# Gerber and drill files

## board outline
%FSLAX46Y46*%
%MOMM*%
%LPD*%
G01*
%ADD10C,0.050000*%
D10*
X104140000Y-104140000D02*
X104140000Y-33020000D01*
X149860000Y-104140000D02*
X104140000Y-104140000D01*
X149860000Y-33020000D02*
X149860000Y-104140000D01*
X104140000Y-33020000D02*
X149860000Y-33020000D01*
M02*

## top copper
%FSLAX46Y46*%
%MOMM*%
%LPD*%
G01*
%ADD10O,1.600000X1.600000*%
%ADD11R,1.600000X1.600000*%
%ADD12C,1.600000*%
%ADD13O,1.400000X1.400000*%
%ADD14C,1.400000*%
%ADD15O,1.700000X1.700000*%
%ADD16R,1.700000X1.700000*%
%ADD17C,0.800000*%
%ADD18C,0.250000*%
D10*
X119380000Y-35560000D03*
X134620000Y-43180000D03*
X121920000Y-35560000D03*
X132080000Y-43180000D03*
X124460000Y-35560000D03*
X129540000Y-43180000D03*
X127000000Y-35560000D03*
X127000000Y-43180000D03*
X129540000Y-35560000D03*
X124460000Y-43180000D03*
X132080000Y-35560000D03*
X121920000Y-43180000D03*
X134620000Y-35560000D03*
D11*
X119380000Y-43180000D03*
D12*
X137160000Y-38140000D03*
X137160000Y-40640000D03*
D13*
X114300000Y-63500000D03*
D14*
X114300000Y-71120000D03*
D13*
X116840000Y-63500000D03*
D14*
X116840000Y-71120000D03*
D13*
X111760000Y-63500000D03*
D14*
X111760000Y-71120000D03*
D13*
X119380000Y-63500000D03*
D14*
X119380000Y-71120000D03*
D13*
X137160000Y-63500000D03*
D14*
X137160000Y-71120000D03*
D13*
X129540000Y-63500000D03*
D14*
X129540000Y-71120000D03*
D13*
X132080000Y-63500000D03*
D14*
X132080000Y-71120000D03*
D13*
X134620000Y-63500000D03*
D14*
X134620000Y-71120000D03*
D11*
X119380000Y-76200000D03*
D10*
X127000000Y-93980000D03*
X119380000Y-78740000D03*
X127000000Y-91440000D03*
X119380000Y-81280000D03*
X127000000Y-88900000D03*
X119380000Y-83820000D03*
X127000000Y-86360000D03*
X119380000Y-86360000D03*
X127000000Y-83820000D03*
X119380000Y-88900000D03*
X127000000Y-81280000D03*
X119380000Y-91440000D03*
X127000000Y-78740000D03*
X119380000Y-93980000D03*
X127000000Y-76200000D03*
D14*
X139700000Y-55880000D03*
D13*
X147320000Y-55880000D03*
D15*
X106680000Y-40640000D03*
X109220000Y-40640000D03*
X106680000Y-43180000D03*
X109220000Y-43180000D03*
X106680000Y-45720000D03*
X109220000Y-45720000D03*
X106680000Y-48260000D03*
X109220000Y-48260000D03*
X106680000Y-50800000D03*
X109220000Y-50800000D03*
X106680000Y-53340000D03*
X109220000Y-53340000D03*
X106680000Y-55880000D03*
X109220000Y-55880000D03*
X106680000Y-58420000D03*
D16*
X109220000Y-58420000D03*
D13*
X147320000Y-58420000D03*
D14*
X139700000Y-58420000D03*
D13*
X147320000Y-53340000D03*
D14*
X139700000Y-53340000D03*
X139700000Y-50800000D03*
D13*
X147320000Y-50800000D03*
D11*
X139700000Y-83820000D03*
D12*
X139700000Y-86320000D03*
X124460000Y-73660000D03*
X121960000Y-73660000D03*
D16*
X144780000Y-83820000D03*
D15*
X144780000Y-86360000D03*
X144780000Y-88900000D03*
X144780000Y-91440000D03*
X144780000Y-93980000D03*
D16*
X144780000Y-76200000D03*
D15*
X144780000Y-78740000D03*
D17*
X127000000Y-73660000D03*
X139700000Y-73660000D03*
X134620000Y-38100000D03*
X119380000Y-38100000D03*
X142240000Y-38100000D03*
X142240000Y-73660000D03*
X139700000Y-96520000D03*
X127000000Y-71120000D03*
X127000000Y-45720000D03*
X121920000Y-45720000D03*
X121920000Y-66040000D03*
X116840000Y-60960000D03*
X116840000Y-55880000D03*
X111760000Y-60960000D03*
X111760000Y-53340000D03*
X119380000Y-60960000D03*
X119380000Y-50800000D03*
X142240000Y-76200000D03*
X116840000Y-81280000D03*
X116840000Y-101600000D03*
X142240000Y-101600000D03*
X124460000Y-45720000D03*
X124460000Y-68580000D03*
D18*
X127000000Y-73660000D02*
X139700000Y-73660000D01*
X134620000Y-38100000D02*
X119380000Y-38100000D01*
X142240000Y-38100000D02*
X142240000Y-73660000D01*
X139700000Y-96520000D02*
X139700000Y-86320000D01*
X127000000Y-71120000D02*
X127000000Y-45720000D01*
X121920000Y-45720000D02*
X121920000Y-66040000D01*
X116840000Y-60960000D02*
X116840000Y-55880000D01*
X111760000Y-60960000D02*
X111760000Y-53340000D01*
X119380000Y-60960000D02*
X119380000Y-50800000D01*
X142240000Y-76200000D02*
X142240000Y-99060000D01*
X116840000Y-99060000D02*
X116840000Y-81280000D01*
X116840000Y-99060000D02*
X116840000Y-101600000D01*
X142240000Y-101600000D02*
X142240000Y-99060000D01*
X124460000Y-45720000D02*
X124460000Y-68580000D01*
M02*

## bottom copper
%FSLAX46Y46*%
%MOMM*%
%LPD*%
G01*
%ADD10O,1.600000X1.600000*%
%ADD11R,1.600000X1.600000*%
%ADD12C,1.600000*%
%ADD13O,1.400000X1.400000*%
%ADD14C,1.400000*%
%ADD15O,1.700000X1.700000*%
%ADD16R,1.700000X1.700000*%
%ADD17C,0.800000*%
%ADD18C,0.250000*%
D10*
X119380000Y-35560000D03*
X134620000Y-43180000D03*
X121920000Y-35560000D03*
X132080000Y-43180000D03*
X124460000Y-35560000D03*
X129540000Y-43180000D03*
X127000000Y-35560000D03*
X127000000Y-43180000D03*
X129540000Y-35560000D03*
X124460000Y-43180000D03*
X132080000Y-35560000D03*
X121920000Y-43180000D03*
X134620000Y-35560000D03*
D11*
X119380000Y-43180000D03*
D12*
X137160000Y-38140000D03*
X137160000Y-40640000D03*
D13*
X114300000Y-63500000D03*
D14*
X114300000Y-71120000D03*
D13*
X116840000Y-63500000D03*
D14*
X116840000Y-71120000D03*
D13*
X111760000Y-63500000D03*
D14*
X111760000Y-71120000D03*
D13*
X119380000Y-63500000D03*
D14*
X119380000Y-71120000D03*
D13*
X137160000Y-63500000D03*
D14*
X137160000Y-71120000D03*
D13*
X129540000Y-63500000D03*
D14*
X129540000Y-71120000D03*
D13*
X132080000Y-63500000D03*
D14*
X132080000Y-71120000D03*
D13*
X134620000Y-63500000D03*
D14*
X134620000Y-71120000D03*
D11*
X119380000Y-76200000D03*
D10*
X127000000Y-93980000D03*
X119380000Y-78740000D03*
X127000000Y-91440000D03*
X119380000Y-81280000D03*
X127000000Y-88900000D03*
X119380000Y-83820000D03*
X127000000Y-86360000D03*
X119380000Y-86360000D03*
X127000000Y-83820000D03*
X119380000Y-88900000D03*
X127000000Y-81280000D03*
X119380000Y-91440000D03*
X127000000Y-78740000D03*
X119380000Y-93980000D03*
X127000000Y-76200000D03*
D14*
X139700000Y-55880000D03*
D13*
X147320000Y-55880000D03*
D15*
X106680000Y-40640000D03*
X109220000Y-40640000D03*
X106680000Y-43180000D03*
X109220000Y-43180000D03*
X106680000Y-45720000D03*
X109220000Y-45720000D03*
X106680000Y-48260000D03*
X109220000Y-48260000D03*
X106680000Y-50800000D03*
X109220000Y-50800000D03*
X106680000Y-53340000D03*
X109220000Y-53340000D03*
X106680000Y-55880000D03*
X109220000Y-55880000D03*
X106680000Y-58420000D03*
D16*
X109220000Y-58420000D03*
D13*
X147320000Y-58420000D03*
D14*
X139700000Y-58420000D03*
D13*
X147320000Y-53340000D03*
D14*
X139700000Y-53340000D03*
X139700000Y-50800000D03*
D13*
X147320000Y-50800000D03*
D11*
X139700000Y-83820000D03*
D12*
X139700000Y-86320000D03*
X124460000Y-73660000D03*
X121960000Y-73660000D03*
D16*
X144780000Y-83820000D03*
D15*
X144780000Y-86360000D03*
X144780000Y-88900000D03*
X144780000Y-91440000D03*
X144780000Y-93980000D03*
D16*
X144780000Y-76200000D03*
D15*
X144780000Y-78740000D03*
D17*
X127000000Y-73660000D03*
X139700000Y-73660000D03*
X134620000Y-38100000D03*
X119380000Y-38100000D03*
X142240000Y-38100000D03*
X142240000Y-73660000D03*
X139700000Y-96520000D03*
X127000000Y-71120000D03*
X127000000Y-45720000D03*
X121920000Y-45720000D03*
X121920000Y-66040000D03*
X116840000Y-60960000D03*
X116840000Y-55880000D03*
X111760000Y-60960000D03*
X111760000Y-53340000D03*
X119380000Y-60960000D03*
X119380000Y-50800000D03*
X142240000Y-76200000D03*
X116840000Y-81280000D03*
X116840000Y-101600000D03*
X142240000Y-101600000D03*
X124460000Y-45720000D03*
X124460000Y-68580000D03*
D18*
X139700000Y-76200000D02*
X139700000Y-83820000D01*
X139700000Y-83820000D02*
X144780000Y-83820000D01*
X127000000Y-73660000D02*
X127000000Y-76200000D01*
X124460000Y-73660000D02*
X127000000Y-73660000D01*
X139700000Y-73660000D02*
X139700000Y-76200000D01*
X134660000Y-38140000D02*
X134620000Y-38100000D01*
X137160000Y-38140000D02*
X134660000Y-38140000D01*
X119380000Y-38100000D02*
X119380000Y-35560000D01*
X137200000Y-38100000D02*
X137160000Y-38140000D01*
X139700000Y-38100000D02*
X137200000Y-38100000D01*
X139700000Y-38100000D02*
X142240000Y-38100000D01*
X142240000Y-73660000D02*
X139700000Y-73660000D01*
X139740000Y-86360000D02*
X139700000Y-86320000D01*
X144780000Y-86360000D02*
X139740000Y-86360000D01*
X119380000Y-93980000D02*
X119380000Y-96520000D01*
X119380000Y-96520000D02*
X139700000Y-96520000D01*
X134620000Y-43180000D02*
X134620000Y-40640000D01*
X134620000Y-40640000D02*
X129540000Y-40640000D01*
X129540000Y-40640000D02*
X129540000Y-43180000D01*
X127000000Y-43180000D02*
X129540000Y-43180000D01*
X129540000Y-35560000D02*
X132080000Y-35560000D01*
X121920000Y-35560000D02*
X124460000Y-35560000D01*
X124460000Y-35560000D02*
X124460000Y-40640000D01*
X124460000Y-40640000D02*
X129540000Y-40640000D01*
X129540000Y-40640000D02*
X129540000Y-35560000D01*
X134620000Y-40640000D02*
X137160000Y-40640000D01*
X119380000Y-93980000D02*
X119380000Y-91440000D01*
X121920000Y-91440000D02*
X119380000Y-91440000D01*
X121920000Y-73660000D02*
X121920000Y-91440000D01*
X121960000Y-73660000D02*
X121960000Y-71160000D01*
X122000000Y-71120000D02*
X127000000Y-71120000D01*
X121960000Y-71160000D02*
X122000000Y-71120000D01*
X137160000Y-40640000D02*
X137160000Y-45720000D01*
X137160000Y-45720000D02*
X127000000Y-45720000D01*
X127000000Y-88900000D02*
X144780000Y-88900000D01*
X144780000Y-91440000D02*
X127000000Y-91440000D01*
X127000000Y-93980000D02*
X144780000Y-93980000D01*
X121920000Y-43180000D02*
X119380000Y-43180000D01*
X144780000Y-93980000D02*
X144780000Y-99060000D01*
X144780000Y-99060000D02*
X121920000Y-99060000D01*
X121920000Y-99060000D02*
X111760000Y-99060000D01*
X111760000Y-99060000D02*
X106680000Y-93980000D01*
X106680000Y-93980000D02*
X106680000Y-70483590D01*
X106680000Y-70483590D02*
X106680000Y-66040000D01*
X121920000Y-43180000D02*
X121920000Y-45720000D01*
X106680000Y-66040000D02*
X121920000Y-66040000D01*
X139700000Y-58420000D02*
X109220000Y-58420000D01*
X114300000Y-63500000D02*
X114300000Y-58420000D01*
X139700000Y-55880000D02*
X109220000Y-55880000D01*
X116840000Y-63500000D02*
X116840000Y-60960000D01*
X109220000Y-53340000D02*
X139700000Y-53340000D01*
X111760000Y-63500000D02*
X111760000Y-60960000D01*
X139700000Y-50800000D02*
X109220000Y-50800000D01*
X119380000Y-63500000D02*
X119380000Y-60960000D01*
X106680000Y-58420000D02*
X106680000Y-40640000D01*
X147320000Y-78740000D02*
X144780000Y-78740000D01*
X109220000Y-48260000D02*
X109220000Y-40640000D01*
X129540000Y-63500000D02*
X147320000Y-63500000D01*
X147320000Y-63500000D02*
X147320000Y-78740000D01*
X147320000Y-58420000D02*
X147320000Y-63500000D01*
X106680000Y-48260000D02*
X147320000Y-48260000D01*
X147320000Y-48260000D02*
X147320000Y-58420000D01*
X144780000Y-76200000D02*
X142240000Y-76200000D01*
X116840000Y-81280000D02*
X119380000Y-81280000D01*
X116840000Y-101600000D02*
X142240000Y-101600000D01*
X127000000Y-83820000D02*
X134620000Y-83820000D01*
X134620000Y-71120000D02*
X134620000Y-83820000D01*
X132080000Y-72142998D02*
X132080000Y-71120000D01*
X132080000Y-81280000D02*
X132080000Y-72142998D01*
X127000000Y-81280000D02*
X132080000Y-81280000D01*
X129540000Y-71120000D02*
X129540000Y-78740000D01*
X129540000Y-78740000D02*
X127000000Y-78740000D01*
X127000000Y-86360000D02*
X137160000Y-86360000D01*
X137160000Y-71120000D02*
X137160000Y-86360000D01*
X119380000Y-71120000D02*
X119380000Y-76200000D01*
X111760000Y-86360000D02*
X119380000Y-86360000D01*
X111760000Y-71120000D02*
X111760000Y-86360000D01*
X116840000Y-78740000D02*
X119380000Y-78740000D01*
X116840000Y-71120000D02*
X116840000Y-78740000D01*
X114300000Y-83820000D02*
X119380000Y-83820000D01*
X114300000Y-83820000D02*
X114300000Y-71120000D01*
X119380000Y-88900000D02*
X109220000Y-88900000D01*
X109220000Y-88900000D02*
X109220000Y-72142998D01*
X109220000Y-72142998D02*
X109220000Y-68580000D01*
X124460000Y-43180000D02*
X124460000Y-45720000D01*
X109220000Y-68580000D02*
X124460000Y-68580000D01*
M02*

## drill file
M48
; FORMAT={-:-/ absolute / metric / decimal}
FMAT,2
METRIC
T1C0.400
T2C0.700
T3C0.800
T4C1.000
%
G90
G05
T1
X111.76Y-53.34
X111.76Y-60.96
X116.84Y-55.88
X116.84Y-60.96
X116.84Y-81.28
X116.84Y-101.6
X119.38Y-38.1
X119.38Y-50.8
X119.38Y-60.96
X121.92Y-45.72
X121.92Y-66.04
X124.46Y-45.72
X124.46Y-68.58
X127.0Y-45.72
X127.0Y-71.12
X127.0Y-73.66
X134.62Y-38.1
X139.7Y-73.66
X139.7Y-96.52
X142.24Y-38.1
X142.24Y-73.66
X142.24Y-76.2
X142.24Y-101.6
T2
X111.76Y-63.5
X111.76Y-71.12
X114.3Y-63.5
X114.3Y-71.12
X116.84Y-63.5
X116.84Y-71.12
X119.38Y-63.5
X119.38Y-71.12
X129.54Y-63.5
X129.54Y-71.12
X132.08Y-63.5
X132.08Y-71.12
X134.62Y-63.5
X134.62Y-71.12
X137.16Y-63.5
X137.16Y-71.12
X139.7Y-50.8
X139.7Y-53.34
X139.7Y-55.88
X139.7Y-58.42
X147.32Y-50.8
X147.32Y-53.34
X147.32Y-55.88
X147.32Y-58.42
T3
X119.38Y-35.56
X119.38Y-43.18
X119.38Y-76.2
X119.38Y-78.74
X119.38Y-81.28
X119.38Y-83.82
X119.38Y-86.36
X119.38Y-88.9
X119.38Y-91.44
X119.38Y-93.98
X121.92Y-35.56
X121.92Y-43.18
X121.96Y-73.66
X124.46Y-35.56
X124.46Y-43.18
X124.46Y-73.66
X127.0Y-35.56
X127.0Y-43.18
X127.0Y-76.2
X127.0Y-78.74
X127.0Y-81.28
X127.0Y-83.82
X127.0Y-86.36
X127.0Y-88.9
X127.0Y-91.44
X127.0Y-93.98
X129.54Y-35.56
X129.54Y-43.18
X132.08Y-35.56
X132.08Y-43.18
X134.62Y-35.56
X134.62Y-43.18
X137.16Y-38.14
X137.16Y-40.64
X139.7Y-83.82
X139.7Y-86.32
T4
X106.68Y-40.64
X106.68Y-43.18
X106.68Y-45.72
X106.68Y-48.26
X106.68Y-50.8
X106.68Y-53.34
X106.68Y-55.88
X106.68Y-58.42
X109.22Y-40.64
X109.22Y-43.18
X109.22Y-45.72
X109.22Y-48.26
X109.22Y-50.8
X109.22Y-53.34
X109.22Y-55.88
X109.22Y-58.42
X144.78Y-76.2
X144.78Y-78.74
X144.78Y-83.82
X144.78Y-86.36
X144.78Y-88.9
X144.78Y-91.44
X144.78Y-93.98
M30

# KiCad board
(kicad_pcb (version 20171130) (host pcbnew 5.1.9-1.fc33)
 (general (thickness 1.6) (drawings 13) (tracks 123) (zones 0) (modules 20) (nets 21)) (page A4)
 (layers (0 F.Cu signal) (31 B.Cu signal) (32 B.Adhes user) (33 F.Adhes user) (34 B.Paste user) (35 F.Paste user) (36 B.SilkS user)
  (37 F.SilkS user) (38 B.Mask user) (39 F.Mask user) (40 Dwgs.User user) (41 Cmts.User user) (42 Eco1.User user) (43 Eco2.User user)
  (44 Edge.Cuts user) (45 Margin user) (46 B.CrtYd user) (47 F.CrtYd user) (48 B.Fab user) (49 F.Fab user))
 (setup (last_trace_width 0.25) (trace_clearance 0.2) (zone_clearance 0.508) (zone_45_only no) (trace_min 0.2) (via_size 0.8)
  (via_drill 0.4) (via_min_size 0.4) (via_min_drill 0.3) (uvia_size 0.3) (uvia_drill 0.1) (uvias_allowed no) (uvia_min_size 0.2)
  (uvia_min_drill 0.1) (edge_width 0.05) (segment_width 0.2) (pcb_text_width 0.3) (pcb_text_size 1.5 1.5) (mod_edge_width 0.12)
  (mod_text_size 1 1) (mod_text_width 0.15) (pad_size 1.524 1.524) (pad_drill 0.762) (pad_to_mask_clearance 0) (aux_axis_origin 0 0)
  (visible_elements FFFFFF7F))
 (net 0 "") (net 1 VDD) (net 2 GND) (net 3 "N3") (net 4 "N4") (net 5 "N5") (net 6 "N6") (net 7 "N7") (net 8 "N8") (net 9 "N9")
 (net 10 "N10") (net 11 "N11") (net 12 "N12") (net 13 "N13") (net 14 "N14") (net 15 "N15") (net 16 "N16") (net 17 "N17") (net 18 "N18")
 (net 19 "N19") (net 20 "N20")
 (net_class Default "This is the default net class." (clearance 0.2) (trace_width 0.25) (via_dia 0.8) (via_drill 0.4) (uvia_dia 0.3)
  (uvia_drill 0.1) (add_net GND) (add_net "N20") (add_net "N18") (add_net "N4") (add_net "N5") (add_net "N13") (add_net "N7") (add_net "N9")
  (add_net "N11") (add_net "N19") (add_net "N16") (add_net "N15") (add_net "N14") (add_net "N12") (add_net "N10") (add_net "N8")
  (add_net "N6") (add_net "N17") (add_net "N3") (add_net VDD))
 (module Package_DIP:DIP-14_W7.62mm (layer F.Cu) (at 119.38 43.18 90)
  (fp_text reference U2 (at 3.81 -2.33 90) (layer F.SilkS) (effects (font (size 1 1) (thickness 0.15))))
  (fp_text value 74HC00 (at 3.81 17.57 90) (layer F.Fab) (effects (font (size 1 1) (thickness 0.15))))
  (pad 14 thru_hole oval (at 7.62 0 90) (size 1.6 1.6) (drill 0.8) (layers *.Cu *.Mask) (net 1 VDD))
  (pad 7 thru_hole oval (at 0 15.24 90) (size 1.6 1.6) (drill 0.8) (layers *.Cu *.Mask) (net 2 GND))
  (pad 13 thru_hole oval (at 7.62 2.54 90) (size 1.6 1.6) (drill 0.8) (layers *.Cu *.Mask) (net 2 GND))
  (pad 6 thru_hole oval (at 0 12.7 90) (size 1.6 1.6) (drill 0.8) (layers *.Cu *.Mask))
  (pad 12 thru_hole oval (at 7.62 5.08 90) (size 1.6 1.6) (drill 0.8) (layers *.Cu *.Mask) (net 2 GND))
  (pad 5 thru_hole oval (at 0 10.16 90) (size 1.6 1.6) (drill 0.8) (layers *.Cu *.Mask) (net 2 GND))
  (pad 11 thru_hole oval (at 7.62 7.62 90) (size 1.6 1.6) (drill 0.8) (layers *.Cu *.Mask))
  (pad 4 thru_hole oval (at 0 7.62 90) (size 1.6 1.6) (drill 0.8) (layers *.Cu *.Mask) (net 2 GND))
  (pad 10 thru_hole oval (at 7.62 10.16 90) (size 1.6 1.6) (drill 0.8) (layers *.Cu *.Mask) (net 2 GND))
  (pad 3 thru_hole oval (at 0 5.08 90) (size 1.6 1.6) (drill 0.8) (layers *.Cu *.Mask) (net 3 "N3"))
  (pad 9 thru_hole oval (at 7.62 12.7 90) (size 1.6 1.6) (drill 0.8) (layers *.Cu *.Mask) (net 2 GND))
  (pad 2 thru_hole oval (at 0 2.54 90) (size 1.6 1.6) (drill 0.8) (layers *.Cu *.Mask) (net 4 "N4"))
  (pad 8 thru_hole oval (at 7.62 15.24 90) (size 1.6 1.6) (drill 0.8) (layers *.Cu *.Mask))
  (pad 1 thru_hole rect (at 0 0 90) (size 1.6 1.6) (drill 0.8) (layers *.Cu *.Mask) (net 4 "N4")))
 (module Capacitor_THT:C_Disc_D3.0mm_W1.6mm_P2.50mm (layer F.Cu) (at 137.16 40.64 90)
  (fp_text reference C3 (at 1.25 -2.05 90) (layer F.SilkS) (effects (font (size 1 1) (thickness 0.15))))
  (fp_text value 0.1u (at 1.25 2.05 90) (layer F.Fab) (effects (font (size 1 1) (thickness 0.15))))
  (pad 2 thru_hole circle (at 2.5 0 90) (size 1.6 1.6) (drill 0.8) (layers *.Cu *.Mask) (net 1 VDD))
  (pad 1 thru_hole circle (at 0 0 90) (size 1.6 1.6) (drill 0.8) (layers *.Cu *.Mask) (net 2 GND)))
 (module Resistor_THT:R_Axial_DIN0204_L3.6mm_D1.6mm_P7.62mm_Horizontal (layer F.Cu) (at 114.3 71.12 90)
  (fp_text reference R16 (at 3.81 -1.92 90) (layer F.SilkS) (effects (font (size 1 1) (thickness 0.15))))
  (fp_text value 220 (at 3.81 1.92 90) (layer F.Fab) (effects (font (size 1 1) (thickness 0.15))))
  (pad 2 thru_hole oval (at 7.62 0 90) (size 1.4 1.4) (drill 0.7) (layers *.Cu *.Mask) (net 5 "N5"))
  (pad 1 thru_hole circle (at 0 0 90) (size 1.4 1.4) (drill 0.7) (layers *.Cu *.Mask) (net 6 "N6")))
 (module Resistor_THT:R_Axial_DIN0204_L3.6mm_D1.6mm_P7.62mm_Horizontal (layer F.Cu) (at 116.84 71.12 90)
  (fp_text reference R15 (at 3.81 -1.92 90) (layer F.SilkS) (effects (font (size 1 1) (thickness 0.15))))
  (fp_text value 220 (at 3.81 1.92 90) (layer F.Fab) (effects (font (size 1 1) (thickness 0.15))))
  (pad 2 thru_hole oval (at 7.62 0 90) (size 1.4 1.4) (drill 0.7) (layers *.Cu *.Mask) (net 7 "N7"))
  (pad 1 thru_hole circle (at 0 0 90) (size 1.4 1.4) (drill 0.7) (layers *.Cu *.Mask) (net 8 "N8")))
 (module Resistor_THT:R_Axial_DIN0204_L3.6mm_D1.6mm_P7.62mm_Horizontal (layer F.Cu) (at 111.76 71.12 90)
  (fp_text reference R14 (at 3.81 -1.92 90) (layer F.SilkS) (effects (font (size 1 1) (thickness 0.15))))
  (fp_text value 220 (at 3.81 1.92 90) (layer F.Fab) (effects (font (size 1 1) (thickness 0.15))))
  (pad 2 thru_hole oval (at 7.62 0 90) (size 1.4 1.4) (drill 0.7) (layers *.Cu *.Mask) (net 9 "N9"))
  (pad 1 thru_hole circle (at 0 0 90) (size 1.4 1.4) (drill 0.7) (layers *.Cu *.Mask) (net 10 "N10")))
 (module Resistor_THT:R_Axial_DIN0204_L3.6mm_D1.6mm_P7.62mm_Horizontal (layer F.Cu) (at 119.38 71.12 90)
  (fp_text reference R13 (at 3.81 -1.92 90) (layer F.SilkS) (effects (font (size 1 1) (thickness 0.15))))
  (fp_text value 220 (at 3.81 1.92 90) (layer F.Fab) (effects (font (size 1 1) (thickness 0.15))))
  (pad 2 thru_hole oval (at 7.62 0 90) (size 1.4 1.4) (drill 0.7) (layers *.Cu *.Mask) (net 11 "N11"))
  (pad 1 thru_hole circle (at 0 0 90) (size 1.4 1.4) (drill 0.7) (layers *.Cu *.Mask) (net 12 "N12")))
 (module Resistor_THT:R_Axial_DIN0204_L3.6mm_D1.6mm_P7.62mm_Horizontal (layer F.Cu) (at 137.16 71.12 90)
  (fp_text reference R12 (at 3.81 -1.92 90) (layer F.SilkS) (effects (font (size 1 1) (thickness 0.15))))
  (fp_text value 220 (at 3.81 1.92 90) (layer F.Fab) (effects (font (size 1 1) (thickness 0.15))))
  (pad 2 thru_hole oval (at 7.62 0 90) (size 1.4 1.4) (drill 0.7) (layers *.Cu *.Mask) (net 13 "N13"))
  (pad 1 thru_hole circle (at 0 0 90) (size 1.4 1.4) (drill 0.7) (layers *.Cu *.Mask) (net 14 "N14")))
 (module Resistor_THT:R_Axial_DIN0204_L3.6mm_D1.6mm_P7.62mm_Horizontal (layer F.Cu) (at 129.54 71.12 90)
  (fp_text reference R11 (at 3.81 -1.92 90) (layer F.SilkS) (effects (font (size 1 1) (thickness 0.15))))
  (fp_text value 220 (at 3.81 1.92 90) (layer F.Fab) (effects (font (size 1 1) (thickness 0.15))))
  (pad 2 thru_hole oval (at 7.62 0 90) (size 1.4 1.4) (drill 0.7) (layers *.Cu *.Mask) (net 13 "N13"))
  (pad 1 thru_hole circle (at 0 0 90) (size 1.4 1.4) (drill 0.7) (layers *.Cu *.Mask) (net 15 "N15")))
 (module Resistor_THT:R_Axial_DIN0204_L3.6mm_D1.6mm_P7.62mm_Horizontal (layer F.Cu) (at 132.08 71.12 90)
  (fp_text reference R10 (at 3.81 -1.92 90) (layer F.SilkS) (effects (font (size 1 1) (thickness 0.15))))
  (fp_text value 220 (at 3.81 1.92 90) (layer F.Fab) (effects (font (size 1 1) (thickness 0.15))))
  (pad 2 thru_hole oval (at 7.62 0 90) (size 1.4 1.4) (drill 0.7) (layers *.Cu *.Mask) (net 13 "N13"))
  (pad 1 thru_hole circle (at 0 0 90) (size 1.4 1.4) (drill 0.7) (layers *.Cu *.Mask) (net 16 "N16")))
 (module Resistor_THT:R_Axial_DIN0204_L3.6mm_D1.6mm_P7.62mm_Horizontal (layer F.Cu) (at 134.62 71.12 90)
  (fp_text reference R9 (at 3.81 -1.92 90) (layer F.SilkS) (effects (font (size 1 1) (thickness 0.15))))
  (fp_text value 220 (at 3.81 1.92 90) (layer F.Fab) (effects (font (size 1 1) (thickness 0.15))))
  (pad 2 thru_hole oval (at 7.62 0 90) (size 1.4 1.4) (drill 0.7) (layers *.Cu *.Mask) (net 13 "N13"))
  (pad 1 thru_hole circle (at 0 0 90) (size 1.4 1.4) (drill 0.7) (layers *.Cu *.Mask) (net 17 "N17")))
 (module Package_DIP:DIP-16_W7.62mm (layer F.Cu) (at 119.38 76.2)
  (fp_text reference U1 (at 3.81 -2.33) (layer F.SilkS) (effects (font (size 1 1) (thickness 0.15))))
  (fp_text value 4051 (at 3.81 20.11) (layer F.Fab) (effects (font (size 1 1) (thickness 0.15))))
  (pad 1 thru_hole rect (at 0 0) (size 1.6 1.6) (drill 0.8) (layers *.Cu *.Mask) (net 12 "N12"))
  (pad 9 thru_hole oval (at 7.62 17.78) (size 1.6 1.6) (drill 0.8) (layers *.Cu *.Mask) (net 4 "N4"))
  (pad 2 thru_hole oval (at 0 2.54) (size 1.6 1.6) (drill 0.8) (layers *.Cu *.Mask) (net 8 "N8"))
  (pad 10 thru_hole oval (at 7.62 15.24) (size 1.6 1.6) (drill 0.8) (layers *.Cu *.Mask) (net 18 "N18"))
  (pad 3 thru_hole oval (at 0 5.08) (size 1.6 1.6) (drill 0.8) (layers *.Cu *.Mask) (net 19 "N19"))
  (pad 11 thru_hole oval (at 7.62 12.7) (size 1.6 1.6) (drill 0.8) (layers *.Cu *.Mask) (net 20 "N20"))
  (pad 4 thru_hole oval (at 0 7.62) (size 1.6 1.6) (drill 0.8) (layers *.Cu *.Mask) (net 6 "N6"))
  (pad 12 thru_hole oval (at 7.62 10.16) (size 1.6 1.6) (drill 0.8) (layers *.Cu *.Mask) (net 14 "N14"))
  (pad 5 thru_hole oval (at 0 10.16) (size 1.6 1.6) (drill 0.8) (layers *.Cu *.Mask) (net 10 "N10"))
  (pad 13 thru_hole oval (at 7.62 7.62) (size 1.6 1.6) (drill 0.8) (layers *.Cu *.Mask) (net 17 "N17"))
  (pad 6 thru_hole oval (at 0 12.7) (size 1.6 1.6) (drill 0.8) (layers *.Cu *.Mask) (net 3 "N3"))
  (pad 14 thru_hole oval (at 7.62 5.08) (size 1.6 1.6) (drill 0.8) (layers *.Cu *.Mask) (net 16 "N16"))
  (pad 7 thru_hole oval (at 0 15.24) (size 1.6 1.6) (drill 0.8) (layers *.Cu *.Mask) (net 2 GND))
  (pad 15 thru_hole oval (at 7.62 2.54) (size 1.6 1.6) (drill 0.8) (layers *.Cu *.Mask) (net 15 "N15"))
  (pad 8 thru_hole oval (at 0 17.78) (size 1.6 1.6) (drill 0.8) (layers *.Cu *.Mask) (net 2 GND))
  (pad 16 thru_hole oval (at 7.62 0) (size 1.6 1.6) (drill 0.8) (layers *.Cu *.Mask) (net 1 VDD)))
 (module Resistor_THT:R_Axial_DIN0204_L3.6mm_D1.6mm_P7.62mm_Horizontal (layer F.Cu) (at 139.7 55.88)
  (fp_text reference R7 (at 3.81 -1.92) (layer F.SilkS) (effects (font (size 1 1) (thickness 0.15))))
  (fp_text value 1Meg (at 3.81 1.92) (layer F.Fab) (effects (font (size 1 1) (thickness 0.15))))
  (pad 1 thru_hole circle (at 0 0) (size 1.4 1.4) (drill 0.7) (layers *.Cu *.Mask) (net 7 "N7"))
  (pad 2 thru_hole oval (at 7.62 0) (size 1.4 1.4) (drill 0.7) (layers *.Cu *.Mask) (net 13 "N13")))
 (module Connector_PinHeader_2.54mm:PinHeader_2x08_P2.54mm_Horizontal (layer F.Cu) (at 109.22 58.42 180)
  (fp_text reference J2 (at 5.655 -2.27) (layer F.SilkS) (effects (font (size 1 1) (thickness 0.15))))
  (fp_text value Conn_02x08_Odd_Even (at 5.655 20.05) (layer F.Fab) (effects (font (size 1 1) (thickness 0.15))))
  (pad 16 thru_hole oval (at 2.54 17.78 180) (size 1.7 1.7) (drill 1) (layers *.Cu *.Mask) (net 13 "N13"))
  (pad 15 thru_hole oval (at 0 17.78 180) (size 1.7 1.7) (drill 1) (layers *.Cu *.Mask) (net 13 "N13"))
  (pad 14 thru_hole oval (at 2.54 15.24 180) (size 1.7 1.7) (drill 1) (layers *.Cu *.Mask) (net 13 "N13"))
  (pad 13 thru_hole oval (at 0 15.24 180) (size 1.7 1.7) (drill 1) (layers *.Cu *.Mask) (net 13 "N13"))
  (pad 12 thru_hole oval (at 2.54 12.7 180) (size 1.7 1.7) (drill 1) (layers *.Cu *.Mask) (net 13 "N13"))
  (pad 11 thru_hole oval (at 0 12.7 180) (size 1.7 1.7) (drill 1) (layers *.Cu *.Mask) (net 13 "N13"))
  (pad 10 thru_hole oval (at 2.54 10.16 180) (size 1.7 1.7) (drill 1) (layers *.Cu *.Mask) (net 13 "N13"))
  (pad 9 thru_hole oval (at 0 10.16 180) (size 1.7 1.7) (drill 1) (layers *.Cu *.Mask) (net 13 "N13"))
  (pad 8 thru_hole oval (at 2.54 7.62 180) (size 1.7 1.7) (drill 1) (layers *.Cu *.Mask) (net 13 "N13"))
  (pad 7 thru_hole oval (at 0 7.62 180) (size 1.7 1.7) (drill 1) (layers *.Cu *.Mask) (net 11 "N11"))
  (pad 6 thru_hole oval (at 2.54 5.08 180) (size 1.7 1.7) (drill 1) (layers *.Cu *.Mask) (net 13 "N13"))
  (pad 5 thru_hole oval (at 0 5.08 180) (size 1.7 1.7) (drill 1) (layers *.Cu *.Mask) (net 9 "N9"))
  (pad 4 thru_hole oval (at 2.54 2.54 180) (size 1.7 1.7) (drill 1) (layers *.Cu *.Mask) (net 13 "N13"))
  (pad 3 thru_hole oval (at 0 2.54 180) (size 1.7 1.7) (drill 1) (layers *.Cu *.Mask) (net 7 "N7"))
  (pad 2 thru_hole oval (at 2.54 0 180) (size 1.7 1.7) (drill 1) (layers *.Cu *.Mask) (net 13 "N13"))
  (pad 1 thru_hole rect (at 0 0 180) (size 1.7 1.7) (drill 1) (layers *.Cu *.Mask) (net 5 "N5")))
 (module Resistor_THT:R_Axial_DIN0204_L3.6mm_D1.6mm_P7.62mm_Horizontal (layer F.Cu) (at 139.7 58.42)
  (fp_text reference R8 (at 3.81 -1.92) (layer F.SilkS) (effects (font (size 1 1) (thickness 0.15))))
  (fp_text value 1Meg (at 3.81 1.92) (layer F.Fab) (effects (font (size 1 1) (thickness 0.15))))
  (pad 2 thru_hole oval (at 7.62 0) (size 1.4 1.4) (drill 0.7) (layers *.Cu *.Mask) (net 13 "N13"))
  (pad 1 thru_hole circle (at 0 0) (size 1.4 1.4) (drill 0.7) (layers *.Cu *.Mask) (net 5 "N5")))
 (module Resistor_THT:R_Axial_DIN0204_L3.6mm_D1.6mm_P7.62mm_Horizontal (layer F.Cu) (at 139.7 53.34)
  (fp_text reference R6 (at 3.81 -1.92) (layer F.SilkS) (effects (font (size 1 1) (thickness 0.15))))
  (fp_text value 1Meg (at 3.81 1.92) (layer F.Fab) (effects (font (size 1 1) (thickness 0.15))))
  (pad 2 thru_hole oval (at 7.62 0) (size 1.4 1.4) (drill 0.7) (layers *.Cu *.Mask) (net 13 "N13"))
  (pad 1 thru_hole circle (at 0 0) (size 1.4 1.4) (drill 0.7) (layers *.Cu *.Mask) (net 9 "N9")))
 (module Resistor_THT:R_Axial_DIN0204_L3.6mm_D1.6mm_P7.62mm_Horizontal (layer F.Cu) (at 139.7 50.8)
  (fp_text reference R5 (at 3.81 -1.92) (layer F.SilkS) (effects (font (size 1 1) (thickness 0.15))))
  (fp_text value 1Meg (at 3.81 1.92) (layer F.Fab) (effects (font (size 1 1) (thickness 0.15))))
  (pad 1 thru_hole circle (at 0 0) (size 1.4 1.4) (drill 0.7) (layers *.Cu *.Mask) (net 11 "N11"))
  (pad 2 thru_hole oval (at 7.62 0) (size 1.4 1.4) (drill 0.7) (layers *.Cu *.Mask) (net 13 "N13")))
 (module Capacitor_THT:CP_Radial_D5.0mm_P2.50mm (layer F.Cu) (at 139.7 83.82 270)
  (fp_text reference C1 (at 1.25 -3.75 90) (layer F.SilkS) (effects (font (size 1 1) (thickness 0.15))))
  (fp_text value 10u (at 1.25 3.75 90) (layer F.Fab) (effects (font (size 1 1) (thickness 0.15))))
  (pad 1 thru_hole rect (at 0 0 270) (size 1.6 1.6) (drill 0.8) (layers *.Cu *.Mask) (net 1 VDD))
  (pad 2 thru_hole circle (at 2.5 0 270) (size 1.6 1.6) (drill 0.8) (layers *.Cu *.Mask) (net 2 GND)))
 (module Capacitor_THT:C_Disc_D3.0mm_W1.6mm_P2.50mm (layer F.Cu) (at 124.46 73.66 180)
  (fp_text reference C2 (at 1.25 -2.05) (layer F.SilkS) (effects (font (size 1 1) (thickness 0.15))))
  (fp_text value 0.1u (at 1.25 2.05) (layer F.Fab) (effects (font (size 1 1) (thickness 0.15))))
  (pad 1 thru_hole circle (at 0 0 180) (size 1.6 1.6) (drill 0.8) (layers *.Cu *.Mask) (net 1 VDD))
  (pad 2 thru_hole circle (at 2.5 0 180) (size 1.6 1.6) (drill 0.8) (layers *.Cu *.Mask) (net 2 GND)))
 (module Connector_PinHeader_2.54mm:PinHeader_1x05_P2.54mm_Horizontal (layer F.Cu) (at 144.78 83.82)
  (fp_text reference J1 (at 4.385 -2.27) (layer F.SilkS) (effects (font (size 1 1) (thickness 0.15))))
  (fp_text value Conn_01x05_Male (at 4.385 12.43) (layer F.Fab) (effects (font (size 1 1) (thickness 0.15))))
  (pad 1 thru_hole rect (at 0 0) (size 1.7 1.7) (drill 1) (layers *.Cu *.Mask) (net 1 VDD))
  (pad 2 thru_hole oval (at 0 2.54) (size 1.7 1.7) (drill 1) (layers *.Cu *.Mask) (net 2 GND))
  (pad 3 thru_hole oval (at 0 5.08) (size 1.7 1.7) (drill 1) (layers *.Cu *.Mask) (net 20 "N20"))
  (pad 4 thru_hole oval (at 0 7.62) (size 1.7 1.7) (drill 1) (layers *.Cu *.Mask) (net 18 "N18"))
  (pad 5 thru_hole oval (at 0 10.16) (size 1.7 1.7) (drill 1) (layers *.Cu *.Mask) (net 4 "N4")))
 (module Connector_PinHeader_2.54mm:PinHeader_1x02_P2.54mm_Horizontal (layer F.Cu) (at 144.78 76.2)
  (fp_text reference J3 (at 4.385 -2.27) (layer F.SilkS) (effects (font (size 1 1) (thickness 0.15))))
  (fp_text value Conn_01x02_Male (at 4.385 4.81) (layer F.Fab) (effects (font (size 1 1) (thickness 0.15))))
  (pad 1 thru_hole rect (at 0 0) (size 1.7 1.7) (drill 1) (layers *.Cu *.Mask) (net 19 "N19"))
  (pad 2 thru_hole oval (at 0 2.54) (size 1.7 1.7) (drill 1) (layers *.Cu *.Mask) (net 13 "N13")))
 (gr_line (start 104.14 104.14) (end 104.14 33.02) (layer Edge.Cuts) (width 0.05))
 (gr_line (start 149.86 104.14) (end 104.14 104.14) (layer Edge.Cuts) (width 0.05))
 (gr_line (start 149.86 33.02) (end 149.86 104.14) (layer Edge.Cuts) (width 0.05))
 (gr_line (start 104.14 33.02) (end 149.86 33.02) (layer Edge.Cuts) (width 0.05))
 (segment (start 139.7 76.2) (end 139.7 83.82) (width 0.25) (layer B.Cu) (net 1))
 (segment (start 139.7 83.82) (end 144.78 83.82) (width 0.25) (layer B.Cu) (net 1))
 (segment (start 127 73.66) (end 127 76.2) (width 0.25) (layer B.Cu) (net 1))
 (via (at 127 73.66) (size 0.8) (drill 0.4) (layers F.Cu B.Cu) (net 1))
 (segment (start 124.46 73.66) (end 127 73.66) (width 0.25) (layer B.Cu) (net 1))
 (via (at 139.7 73.66) (size 0.8) (drill 0.4) (layers F.Cu B.Cu) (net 1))
 (segment (start 127 73.66) (end 139.7 73.66) (width 0.25) (layer F.Cu) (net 1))
 (segment (start 139.7 73.66) (end 139.7 76.2) (width 0.25) (layer B.Cu) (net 1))
 (segment (start 134.66 38.14) (end 134.62 38.1) (width 0.25) (layer B.Cu) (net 1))
 (via (at 134.62 38.1) (size 0.8) (drill 0.4) (layers F.Cu B.Cu) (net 1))
 (segment (start 137.16 38.14) (end 134.66 38.14) (width 0.25) (layer B.Cu) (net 1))
 (via (at 119.38 38.1) (size 0.8) (drill 0.4) (layers F.Cu B.Cu) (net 1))
 (segment (start 134.62 38.1) (end 119.38 38.1) (width 0.25) (layer F.Cu) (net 1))
 (segment (start 119.38 38.1) (end 119.38 35.56) (width 0.25) (layer B.Cu) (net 1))
 (segment (start 137.2 38.1) (end 137.16 38.14) (width 0.25) (layer B.Cu) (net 1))
 (segment (start 139.7 38.1) (end 137.2 38.1) (width 0.25) (layer B.Cu) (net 1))
 (via (at 142.24 38.1) (size 0.8) (drill 0.4) (layers F.Cu B.Cu) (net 1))
 (segment (start 139.7 38.1) (end 142.24 38.1) (width 0.25) (layer B.Cu) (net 1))
 (via (at 142.24 73.66) (size 0.8) (drill 0.4) (layers F.Cu B.Cu) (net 1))
 (segment (start 142.24 38.1) (end 142.24 73.66) (width 0.25) (layer F.Cu) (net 1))
 (segment (start 142.24 73.66) (end 139.7 73.66) (width 0.25) (layer B.Cu) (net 1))
 (segment (start 139.74 86.36) (end 139.7 86.32) (width 0.25) (layer B.Cu) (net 2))
 (segment (start 144.78 86.36) (end 139.74 86.36) (width 0.25) (layer B.Cu) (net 2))
 (segment (start 119.38 93.98) (end 119.38 96.52) (width 0.25) (layer B.Cu) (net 2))
 (via (at 139.7 96.52) (size 0.8) (drill 0.4) (layers F.Cu B.Cu) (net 2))
 (segment (start 119.38 96.52) (end 139.7 96.52) (width 0.25) (layer B.Cu) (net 2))
 (segment (start 139.7 96.52) (end 139.7 86.32) (width 0.25) (layer F.Cu) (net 2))
 (segment (start 134.62 43.18) (end 134.62 40.64) (width 0.25) (layer B.Cu) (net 2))
 (segment (start 134.62 40.64) (end 129.54 40.64) (width 0.25) (layer B.Cu) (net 2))
 (segment (start 129.54 40.64) (end 129.54 43.18) (width 0.25) (layer B.Cu) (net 2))
 (segment (start 127 43.18) (end 129.54 43.18) (width 0.25) (layer B.Cu) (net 2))
 (segment (start 129.54 35.56) (end 132.08 35.56) (width 0.25) (layer B.Cu) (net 2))
 (segment (start 121.92 35.56) (end 124.46 35.56) (width 0.25) (layer B.Cu) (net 2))
 (segment (start 124.46 35.56) (end 124.46 40.64) (width 0.25) (layer B.Cu) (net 2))
 (segment (start 124.46 40.64) (end 129.54 40.64) (width 0.25) (layer B.Cu) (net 2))
 (segment (start 129.54 40.64) (end 129.54 35.56) (width 0.25) (layer B.Cu) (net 2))
 (segment (start 134.62 40.64) (end 137.16 40.64) (width 0.25) (layer B.Cu) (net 2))
 (segment (start 119.38 93.98) (end 119.38 91.44) (width 0.25) (layer B.Cu) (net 2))
 (segment (start 121.92 91.44) (end 119.38 91.44) (width 0.25) (layer B.Cu) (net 2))
 (segment (start 121.92 73.66) (end 121.92 91.44) (width 0.25) (layer B.Cu) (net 2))
 (segment (start 121.96 73.66) (end 121.96 71.16) (width 0.25) (layer B.Cu) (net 2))
 (via (at 127 71.12) (size 0.8) (drill 0.4) (layers F.Cu B.Cu) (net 2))
 (segment (start 122 71.12) (end 127 71.12) (width 0.25) (layer B.Cu) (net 2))
 (segment (start 121.96 71.16) (end 122 71.12) (width 0.25) (layer B.Cu) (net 2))
 (via (at 127 45.72) (size 0.8) (drill 0.4) (layers F.Cu B.Cu) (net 2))
 (segment (start 127 71.12) (end 127 45.72) (width 0.25) (layer F.Cu) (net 2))
 (segment (start 137.16 40.64) (end 137.16 45.72) (width 0.25) (layer B.Cu) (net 2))
 (segment (start 137.16 45.72) (end 127 45.72) (width 0.25) (layer B.Cu) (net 2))
 (segment (start 127 88.9) (end 144.78 88.9) (width 0.25) (layer B.Cu) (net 20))
 (segment (start 144.78 91.44) (end 127 91.44) (width 0.25) (layer B.Cu) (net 18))
 (segment (start 127 93.98) (end 144.78 93.98) (width 0.25) (layer B.Cu) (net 4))
 (segment (start 121.92 43.18) (end 119.38 43.18) (width 0.25) (layer B.Cu) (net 4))
 (segment (start 144.78 93.98) (end 144.78 99.06) (width 0.25) (layer B.Cu) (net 4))
 (segment (start 144.78 99.06) (end 121.92 99.06) (width 0.25) (layer B.Cu) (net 4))
 (segment (start 121.92 99.06) (end 111.76 99.06) (width 0.25) (layer B.Cu) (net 4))
 (segment (start 111.76 99.06) (end 106.68 93.98) (width 0.25) (layer B.Cu) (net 4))
 (segment (start 106.68 93.98) (end 106.68 70.48359) (width 0.25) (layer B.Cu) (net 4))
 (segment (start 106.68 70.48359) (end 106.68 66.04) (width 0.25) (layer B.Cu) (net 4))
 (via (at 121.92 45.72) (size 0.8) (drill 0.4) (layers F.Cu B.Cu) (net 4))
 (segment (start 121.92 43.18) (end 121.92 45.72) (width 0.25) (layer B.Cu) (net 4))
 (segment (start 121.92 45.72) (end 121.92 66.04) (width 0.25) (layer F.Cu) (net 4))
 (via (at 121.92 66.04) (size 0.8) (drill 0.4) (layers F.Cu B.Cu) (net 4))
 (segment (start 106.68 66.04) (end 121.92 66.04) (width 0.25) (layer B.Cu) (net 4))
 (segment (start 139.7 58.42) (end 109.22 58.42) (width 0.25) (layer B.Cu) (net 5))
 (segment (start 114.3 63.5) (end 114.3 58.42) (width 0.25) (layer B.Cu) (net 5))
 (segment (start 139.7 55.88) (end 109.22 55.88) (width 0.25) (layer B.Cu) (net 7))
 (via (at 116.84 60.96) (size 0.8) (drill 0.4) (layers F.Cu B.Cu) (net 7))
 (segment (start 116.84 63.5) (end 116.84 60.96) (width 0.25) (layer B.Cu) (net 7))
 (via (at 116.84 55.88) (size 0.8) (drill 0.4) (layers F.Cu B.Cu) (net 7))
 (segment (start 116.84 60.96) (end 116.84 55.88) (width 0.25) (layer F.Cu) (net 7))
 (segment (start 109.22 53.34) (end 139.7 53.34) (width 0.25) (layer B.Cu) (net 9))
 (via (at 111.76 60.96) (size 0.8) (drill 0.4) (layers F.Cu B.Cu) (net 9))
 (segment (start 111.76 63.5) (end 111.76 60.96) (width 0.25) (layer B.Cu) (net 9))
 (segment (start 111.76 60.96) (end 111.76 53.34) (width 0.25) (layer F.Cu) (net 9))
 (via (at 111.76 53.34) (size 0.8) (drill 0.4) (layers F.Cu B.Cu) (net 9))
 (segment (start 139.7 50.8) (end 109.22 50.8) (width 0.25) (layer B.Cu) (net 11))
 (via (at 119.38 60.96) (size 0.8) (drill 0.4) (layers F.Cu B.Cu) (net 11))
 (segment (start 119.38 63.5) (end 119.38 60.96) (width 0.25) (layer B.Cu) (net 11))
 (via (at 119.38 50.8) (size 0.8) (drill 0.4) (layers F.Cu B.Cu) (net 11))
 (segment (start 119.38 60.96) (end 119.38 50.8) (width 0.25) (layer F.Cu) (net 11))
 (segment (start 106.68 58.42) (end 106.68 40.64) (width 0.25) (layer B.Cu) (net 13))
 (segment (start 147.32 78.74) (end 144.78 78.74) (width 0.25) (layer B.Cu) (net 13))
 (segment (start 109.22 48.26) (end 109.22 40.64) (width 0.25) (layer B.Cu) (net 13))
 (segment (start 129.54 63.5) (end 147.32 63.5) (width 0.25) (layer B.Cu) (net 13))
 (segment (start 147.32 63.5) (end 147.32 78.74) (width 0.25) (layer B.Cu) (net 13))
 (segment (start 147.32 58.42) (end 147.32 63.5) (width 0.25) (layer B.Cu) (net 13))
 (segment (start 106.68 48.26) (end 147.32 48.26) (width 0.25) (layer B.Cu) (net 13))
 (segment (start 147.32 48.26) (end 147.32 58.42) (width 0.25) (layer B.Cu) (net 13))
 (via (at 142.24 76.2) (size 0.8) (drill 0.4) (layers F.Cu B.Cu) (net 19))
 (segment (start 144.78 76.2) (end 142.24 76.2) (width 0.25) (layer B.Cu) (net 19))
 (segment (start 142.24 76.2) (end 142.24 99.06) (width 0.25) (layer F.Cu) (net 19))
 (via (at 116.84 81.28) (size 0.8) (drill 0.4) (layers F.Cu B.Cu) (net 19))
 (segment (start 116.84 99.06) (end 116.84 81.28) (width 0.25) (layer F.Cu) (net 19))
 (segment (start 116.84 81.28) (end 119.38 81.28) (width 0.25) (layer B.Cu) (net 19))
 (via (at 116.84 101.6) (size 0.8) (drill 0.4) (layers F.Cu B.Cu) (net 19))
 (segment (start 116.84 99.06) (end 116.84 101.6) (width 0.25) (layer F.Cu) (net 19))
 (via (at 142.24 101.6) (size 0.8) (drill 0.4) (layers F.Cu B.Cu) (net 19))
 (segment (start 116.84 101.6) (end 142.24 101.6) (width 0.25) (layer B.Cu) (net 19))
 (segment (start 142.24 101.6) (end 142.24 99.06) (width 0.25) (layer F.Cu) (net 19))
 (segment (start 127 83.82) (end 134.62 83.82) (width 0.25) (layer B.Cu) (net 17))
 (segment (start 134.62 71.12) (end 134.62 83.82) (width 0.25) (layer B.Cu) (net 17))
 (segment (start 132.08 72.142998) (end 132.08 71.12) (width 0.25) (layer B.Cu) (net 16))
 (segment (start 132.08 81.28) (end 132.08 72.142998) (width 0.25) (layer B.Cu) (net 16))
 (segment (start 127 81.28) (end 132.08 81.28) (width 0.25) (layer B.Cu) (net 16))
 (segment (start 129.54 71.12) (end 129.54 78.74) (width 0.25) (layer B.Cu) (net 15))
 (segment (start 129.54 78.74) (end 127 78.74) (width 0.25) (layer B.Cu) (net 15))
 (segment (start 127 86.36) (end 137.16 86.36) (width 0.25) (layer B.Cu) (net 14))
 (segment (start 137.16 71.12) (end 137.16 86.36) (width 0.25) (layer B.Cu) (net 14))
 (segment (start 119.38 71.12) (end 119.38 76.2) (width 0.25) (layer B.Cu) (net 12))
 (segment (start 111.76 86.36) (end 119.38 86.36) (width 0.25) (layer B.Cu) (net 10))
 (segment (start 111.76 71.12) (end 111.76 86.36) (width 0.25) (layer B.Cu) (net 10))
 (segment (start 116.84 78.74) (end 119.38 78.74) (width 0.25) (layer B.Cu) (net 8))
 (segment (start 116.84 71.12) (end 116.84 78.74) (width 0.25) (layer B.Cu) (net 8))
 (segment (start 114.3 83.82) (end 119.38 83.82) (width 0.25) (layer B.Cu) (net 6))
 (segment (start 114.3 83.82) (end 114.3 71.12) (width 0.25) (layer B.Cu) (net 6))
 (segment (start 119.38 88.9) (end 109.22 88.9) (width 0.25) (layer B.Cu) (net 3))
 (segment (start 109.22 88.9) (end 109.22 72.142998) (width 0.25) (layer B.Cu) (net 3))
 (segment (start 109.22 72.142998) (end 109.22 68.58) (width 0.25) (layer B.Cu) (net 3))
 (via (at 124.46 45.72) (size 0.8) (drill 0.4) (layers F.Cu B.Cu) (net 3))
 (segment (start 124.46 43.18) (end 124.46 45.72) (width 0.25) (layer B.Cu) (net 3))
 (segment (start 124.46 45.72) (end 124.46 68.58) (width 0.25) (layer F.Cu) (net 3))
 (via (at 124.46 68.58) (size 0.8) (drill 0.4) (layers F.Cu B.Cu) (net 3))
 (segment (start 109.22 68.58) (end 124.46 68.58) (width 0.25) (layer B.Cu) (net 3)))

